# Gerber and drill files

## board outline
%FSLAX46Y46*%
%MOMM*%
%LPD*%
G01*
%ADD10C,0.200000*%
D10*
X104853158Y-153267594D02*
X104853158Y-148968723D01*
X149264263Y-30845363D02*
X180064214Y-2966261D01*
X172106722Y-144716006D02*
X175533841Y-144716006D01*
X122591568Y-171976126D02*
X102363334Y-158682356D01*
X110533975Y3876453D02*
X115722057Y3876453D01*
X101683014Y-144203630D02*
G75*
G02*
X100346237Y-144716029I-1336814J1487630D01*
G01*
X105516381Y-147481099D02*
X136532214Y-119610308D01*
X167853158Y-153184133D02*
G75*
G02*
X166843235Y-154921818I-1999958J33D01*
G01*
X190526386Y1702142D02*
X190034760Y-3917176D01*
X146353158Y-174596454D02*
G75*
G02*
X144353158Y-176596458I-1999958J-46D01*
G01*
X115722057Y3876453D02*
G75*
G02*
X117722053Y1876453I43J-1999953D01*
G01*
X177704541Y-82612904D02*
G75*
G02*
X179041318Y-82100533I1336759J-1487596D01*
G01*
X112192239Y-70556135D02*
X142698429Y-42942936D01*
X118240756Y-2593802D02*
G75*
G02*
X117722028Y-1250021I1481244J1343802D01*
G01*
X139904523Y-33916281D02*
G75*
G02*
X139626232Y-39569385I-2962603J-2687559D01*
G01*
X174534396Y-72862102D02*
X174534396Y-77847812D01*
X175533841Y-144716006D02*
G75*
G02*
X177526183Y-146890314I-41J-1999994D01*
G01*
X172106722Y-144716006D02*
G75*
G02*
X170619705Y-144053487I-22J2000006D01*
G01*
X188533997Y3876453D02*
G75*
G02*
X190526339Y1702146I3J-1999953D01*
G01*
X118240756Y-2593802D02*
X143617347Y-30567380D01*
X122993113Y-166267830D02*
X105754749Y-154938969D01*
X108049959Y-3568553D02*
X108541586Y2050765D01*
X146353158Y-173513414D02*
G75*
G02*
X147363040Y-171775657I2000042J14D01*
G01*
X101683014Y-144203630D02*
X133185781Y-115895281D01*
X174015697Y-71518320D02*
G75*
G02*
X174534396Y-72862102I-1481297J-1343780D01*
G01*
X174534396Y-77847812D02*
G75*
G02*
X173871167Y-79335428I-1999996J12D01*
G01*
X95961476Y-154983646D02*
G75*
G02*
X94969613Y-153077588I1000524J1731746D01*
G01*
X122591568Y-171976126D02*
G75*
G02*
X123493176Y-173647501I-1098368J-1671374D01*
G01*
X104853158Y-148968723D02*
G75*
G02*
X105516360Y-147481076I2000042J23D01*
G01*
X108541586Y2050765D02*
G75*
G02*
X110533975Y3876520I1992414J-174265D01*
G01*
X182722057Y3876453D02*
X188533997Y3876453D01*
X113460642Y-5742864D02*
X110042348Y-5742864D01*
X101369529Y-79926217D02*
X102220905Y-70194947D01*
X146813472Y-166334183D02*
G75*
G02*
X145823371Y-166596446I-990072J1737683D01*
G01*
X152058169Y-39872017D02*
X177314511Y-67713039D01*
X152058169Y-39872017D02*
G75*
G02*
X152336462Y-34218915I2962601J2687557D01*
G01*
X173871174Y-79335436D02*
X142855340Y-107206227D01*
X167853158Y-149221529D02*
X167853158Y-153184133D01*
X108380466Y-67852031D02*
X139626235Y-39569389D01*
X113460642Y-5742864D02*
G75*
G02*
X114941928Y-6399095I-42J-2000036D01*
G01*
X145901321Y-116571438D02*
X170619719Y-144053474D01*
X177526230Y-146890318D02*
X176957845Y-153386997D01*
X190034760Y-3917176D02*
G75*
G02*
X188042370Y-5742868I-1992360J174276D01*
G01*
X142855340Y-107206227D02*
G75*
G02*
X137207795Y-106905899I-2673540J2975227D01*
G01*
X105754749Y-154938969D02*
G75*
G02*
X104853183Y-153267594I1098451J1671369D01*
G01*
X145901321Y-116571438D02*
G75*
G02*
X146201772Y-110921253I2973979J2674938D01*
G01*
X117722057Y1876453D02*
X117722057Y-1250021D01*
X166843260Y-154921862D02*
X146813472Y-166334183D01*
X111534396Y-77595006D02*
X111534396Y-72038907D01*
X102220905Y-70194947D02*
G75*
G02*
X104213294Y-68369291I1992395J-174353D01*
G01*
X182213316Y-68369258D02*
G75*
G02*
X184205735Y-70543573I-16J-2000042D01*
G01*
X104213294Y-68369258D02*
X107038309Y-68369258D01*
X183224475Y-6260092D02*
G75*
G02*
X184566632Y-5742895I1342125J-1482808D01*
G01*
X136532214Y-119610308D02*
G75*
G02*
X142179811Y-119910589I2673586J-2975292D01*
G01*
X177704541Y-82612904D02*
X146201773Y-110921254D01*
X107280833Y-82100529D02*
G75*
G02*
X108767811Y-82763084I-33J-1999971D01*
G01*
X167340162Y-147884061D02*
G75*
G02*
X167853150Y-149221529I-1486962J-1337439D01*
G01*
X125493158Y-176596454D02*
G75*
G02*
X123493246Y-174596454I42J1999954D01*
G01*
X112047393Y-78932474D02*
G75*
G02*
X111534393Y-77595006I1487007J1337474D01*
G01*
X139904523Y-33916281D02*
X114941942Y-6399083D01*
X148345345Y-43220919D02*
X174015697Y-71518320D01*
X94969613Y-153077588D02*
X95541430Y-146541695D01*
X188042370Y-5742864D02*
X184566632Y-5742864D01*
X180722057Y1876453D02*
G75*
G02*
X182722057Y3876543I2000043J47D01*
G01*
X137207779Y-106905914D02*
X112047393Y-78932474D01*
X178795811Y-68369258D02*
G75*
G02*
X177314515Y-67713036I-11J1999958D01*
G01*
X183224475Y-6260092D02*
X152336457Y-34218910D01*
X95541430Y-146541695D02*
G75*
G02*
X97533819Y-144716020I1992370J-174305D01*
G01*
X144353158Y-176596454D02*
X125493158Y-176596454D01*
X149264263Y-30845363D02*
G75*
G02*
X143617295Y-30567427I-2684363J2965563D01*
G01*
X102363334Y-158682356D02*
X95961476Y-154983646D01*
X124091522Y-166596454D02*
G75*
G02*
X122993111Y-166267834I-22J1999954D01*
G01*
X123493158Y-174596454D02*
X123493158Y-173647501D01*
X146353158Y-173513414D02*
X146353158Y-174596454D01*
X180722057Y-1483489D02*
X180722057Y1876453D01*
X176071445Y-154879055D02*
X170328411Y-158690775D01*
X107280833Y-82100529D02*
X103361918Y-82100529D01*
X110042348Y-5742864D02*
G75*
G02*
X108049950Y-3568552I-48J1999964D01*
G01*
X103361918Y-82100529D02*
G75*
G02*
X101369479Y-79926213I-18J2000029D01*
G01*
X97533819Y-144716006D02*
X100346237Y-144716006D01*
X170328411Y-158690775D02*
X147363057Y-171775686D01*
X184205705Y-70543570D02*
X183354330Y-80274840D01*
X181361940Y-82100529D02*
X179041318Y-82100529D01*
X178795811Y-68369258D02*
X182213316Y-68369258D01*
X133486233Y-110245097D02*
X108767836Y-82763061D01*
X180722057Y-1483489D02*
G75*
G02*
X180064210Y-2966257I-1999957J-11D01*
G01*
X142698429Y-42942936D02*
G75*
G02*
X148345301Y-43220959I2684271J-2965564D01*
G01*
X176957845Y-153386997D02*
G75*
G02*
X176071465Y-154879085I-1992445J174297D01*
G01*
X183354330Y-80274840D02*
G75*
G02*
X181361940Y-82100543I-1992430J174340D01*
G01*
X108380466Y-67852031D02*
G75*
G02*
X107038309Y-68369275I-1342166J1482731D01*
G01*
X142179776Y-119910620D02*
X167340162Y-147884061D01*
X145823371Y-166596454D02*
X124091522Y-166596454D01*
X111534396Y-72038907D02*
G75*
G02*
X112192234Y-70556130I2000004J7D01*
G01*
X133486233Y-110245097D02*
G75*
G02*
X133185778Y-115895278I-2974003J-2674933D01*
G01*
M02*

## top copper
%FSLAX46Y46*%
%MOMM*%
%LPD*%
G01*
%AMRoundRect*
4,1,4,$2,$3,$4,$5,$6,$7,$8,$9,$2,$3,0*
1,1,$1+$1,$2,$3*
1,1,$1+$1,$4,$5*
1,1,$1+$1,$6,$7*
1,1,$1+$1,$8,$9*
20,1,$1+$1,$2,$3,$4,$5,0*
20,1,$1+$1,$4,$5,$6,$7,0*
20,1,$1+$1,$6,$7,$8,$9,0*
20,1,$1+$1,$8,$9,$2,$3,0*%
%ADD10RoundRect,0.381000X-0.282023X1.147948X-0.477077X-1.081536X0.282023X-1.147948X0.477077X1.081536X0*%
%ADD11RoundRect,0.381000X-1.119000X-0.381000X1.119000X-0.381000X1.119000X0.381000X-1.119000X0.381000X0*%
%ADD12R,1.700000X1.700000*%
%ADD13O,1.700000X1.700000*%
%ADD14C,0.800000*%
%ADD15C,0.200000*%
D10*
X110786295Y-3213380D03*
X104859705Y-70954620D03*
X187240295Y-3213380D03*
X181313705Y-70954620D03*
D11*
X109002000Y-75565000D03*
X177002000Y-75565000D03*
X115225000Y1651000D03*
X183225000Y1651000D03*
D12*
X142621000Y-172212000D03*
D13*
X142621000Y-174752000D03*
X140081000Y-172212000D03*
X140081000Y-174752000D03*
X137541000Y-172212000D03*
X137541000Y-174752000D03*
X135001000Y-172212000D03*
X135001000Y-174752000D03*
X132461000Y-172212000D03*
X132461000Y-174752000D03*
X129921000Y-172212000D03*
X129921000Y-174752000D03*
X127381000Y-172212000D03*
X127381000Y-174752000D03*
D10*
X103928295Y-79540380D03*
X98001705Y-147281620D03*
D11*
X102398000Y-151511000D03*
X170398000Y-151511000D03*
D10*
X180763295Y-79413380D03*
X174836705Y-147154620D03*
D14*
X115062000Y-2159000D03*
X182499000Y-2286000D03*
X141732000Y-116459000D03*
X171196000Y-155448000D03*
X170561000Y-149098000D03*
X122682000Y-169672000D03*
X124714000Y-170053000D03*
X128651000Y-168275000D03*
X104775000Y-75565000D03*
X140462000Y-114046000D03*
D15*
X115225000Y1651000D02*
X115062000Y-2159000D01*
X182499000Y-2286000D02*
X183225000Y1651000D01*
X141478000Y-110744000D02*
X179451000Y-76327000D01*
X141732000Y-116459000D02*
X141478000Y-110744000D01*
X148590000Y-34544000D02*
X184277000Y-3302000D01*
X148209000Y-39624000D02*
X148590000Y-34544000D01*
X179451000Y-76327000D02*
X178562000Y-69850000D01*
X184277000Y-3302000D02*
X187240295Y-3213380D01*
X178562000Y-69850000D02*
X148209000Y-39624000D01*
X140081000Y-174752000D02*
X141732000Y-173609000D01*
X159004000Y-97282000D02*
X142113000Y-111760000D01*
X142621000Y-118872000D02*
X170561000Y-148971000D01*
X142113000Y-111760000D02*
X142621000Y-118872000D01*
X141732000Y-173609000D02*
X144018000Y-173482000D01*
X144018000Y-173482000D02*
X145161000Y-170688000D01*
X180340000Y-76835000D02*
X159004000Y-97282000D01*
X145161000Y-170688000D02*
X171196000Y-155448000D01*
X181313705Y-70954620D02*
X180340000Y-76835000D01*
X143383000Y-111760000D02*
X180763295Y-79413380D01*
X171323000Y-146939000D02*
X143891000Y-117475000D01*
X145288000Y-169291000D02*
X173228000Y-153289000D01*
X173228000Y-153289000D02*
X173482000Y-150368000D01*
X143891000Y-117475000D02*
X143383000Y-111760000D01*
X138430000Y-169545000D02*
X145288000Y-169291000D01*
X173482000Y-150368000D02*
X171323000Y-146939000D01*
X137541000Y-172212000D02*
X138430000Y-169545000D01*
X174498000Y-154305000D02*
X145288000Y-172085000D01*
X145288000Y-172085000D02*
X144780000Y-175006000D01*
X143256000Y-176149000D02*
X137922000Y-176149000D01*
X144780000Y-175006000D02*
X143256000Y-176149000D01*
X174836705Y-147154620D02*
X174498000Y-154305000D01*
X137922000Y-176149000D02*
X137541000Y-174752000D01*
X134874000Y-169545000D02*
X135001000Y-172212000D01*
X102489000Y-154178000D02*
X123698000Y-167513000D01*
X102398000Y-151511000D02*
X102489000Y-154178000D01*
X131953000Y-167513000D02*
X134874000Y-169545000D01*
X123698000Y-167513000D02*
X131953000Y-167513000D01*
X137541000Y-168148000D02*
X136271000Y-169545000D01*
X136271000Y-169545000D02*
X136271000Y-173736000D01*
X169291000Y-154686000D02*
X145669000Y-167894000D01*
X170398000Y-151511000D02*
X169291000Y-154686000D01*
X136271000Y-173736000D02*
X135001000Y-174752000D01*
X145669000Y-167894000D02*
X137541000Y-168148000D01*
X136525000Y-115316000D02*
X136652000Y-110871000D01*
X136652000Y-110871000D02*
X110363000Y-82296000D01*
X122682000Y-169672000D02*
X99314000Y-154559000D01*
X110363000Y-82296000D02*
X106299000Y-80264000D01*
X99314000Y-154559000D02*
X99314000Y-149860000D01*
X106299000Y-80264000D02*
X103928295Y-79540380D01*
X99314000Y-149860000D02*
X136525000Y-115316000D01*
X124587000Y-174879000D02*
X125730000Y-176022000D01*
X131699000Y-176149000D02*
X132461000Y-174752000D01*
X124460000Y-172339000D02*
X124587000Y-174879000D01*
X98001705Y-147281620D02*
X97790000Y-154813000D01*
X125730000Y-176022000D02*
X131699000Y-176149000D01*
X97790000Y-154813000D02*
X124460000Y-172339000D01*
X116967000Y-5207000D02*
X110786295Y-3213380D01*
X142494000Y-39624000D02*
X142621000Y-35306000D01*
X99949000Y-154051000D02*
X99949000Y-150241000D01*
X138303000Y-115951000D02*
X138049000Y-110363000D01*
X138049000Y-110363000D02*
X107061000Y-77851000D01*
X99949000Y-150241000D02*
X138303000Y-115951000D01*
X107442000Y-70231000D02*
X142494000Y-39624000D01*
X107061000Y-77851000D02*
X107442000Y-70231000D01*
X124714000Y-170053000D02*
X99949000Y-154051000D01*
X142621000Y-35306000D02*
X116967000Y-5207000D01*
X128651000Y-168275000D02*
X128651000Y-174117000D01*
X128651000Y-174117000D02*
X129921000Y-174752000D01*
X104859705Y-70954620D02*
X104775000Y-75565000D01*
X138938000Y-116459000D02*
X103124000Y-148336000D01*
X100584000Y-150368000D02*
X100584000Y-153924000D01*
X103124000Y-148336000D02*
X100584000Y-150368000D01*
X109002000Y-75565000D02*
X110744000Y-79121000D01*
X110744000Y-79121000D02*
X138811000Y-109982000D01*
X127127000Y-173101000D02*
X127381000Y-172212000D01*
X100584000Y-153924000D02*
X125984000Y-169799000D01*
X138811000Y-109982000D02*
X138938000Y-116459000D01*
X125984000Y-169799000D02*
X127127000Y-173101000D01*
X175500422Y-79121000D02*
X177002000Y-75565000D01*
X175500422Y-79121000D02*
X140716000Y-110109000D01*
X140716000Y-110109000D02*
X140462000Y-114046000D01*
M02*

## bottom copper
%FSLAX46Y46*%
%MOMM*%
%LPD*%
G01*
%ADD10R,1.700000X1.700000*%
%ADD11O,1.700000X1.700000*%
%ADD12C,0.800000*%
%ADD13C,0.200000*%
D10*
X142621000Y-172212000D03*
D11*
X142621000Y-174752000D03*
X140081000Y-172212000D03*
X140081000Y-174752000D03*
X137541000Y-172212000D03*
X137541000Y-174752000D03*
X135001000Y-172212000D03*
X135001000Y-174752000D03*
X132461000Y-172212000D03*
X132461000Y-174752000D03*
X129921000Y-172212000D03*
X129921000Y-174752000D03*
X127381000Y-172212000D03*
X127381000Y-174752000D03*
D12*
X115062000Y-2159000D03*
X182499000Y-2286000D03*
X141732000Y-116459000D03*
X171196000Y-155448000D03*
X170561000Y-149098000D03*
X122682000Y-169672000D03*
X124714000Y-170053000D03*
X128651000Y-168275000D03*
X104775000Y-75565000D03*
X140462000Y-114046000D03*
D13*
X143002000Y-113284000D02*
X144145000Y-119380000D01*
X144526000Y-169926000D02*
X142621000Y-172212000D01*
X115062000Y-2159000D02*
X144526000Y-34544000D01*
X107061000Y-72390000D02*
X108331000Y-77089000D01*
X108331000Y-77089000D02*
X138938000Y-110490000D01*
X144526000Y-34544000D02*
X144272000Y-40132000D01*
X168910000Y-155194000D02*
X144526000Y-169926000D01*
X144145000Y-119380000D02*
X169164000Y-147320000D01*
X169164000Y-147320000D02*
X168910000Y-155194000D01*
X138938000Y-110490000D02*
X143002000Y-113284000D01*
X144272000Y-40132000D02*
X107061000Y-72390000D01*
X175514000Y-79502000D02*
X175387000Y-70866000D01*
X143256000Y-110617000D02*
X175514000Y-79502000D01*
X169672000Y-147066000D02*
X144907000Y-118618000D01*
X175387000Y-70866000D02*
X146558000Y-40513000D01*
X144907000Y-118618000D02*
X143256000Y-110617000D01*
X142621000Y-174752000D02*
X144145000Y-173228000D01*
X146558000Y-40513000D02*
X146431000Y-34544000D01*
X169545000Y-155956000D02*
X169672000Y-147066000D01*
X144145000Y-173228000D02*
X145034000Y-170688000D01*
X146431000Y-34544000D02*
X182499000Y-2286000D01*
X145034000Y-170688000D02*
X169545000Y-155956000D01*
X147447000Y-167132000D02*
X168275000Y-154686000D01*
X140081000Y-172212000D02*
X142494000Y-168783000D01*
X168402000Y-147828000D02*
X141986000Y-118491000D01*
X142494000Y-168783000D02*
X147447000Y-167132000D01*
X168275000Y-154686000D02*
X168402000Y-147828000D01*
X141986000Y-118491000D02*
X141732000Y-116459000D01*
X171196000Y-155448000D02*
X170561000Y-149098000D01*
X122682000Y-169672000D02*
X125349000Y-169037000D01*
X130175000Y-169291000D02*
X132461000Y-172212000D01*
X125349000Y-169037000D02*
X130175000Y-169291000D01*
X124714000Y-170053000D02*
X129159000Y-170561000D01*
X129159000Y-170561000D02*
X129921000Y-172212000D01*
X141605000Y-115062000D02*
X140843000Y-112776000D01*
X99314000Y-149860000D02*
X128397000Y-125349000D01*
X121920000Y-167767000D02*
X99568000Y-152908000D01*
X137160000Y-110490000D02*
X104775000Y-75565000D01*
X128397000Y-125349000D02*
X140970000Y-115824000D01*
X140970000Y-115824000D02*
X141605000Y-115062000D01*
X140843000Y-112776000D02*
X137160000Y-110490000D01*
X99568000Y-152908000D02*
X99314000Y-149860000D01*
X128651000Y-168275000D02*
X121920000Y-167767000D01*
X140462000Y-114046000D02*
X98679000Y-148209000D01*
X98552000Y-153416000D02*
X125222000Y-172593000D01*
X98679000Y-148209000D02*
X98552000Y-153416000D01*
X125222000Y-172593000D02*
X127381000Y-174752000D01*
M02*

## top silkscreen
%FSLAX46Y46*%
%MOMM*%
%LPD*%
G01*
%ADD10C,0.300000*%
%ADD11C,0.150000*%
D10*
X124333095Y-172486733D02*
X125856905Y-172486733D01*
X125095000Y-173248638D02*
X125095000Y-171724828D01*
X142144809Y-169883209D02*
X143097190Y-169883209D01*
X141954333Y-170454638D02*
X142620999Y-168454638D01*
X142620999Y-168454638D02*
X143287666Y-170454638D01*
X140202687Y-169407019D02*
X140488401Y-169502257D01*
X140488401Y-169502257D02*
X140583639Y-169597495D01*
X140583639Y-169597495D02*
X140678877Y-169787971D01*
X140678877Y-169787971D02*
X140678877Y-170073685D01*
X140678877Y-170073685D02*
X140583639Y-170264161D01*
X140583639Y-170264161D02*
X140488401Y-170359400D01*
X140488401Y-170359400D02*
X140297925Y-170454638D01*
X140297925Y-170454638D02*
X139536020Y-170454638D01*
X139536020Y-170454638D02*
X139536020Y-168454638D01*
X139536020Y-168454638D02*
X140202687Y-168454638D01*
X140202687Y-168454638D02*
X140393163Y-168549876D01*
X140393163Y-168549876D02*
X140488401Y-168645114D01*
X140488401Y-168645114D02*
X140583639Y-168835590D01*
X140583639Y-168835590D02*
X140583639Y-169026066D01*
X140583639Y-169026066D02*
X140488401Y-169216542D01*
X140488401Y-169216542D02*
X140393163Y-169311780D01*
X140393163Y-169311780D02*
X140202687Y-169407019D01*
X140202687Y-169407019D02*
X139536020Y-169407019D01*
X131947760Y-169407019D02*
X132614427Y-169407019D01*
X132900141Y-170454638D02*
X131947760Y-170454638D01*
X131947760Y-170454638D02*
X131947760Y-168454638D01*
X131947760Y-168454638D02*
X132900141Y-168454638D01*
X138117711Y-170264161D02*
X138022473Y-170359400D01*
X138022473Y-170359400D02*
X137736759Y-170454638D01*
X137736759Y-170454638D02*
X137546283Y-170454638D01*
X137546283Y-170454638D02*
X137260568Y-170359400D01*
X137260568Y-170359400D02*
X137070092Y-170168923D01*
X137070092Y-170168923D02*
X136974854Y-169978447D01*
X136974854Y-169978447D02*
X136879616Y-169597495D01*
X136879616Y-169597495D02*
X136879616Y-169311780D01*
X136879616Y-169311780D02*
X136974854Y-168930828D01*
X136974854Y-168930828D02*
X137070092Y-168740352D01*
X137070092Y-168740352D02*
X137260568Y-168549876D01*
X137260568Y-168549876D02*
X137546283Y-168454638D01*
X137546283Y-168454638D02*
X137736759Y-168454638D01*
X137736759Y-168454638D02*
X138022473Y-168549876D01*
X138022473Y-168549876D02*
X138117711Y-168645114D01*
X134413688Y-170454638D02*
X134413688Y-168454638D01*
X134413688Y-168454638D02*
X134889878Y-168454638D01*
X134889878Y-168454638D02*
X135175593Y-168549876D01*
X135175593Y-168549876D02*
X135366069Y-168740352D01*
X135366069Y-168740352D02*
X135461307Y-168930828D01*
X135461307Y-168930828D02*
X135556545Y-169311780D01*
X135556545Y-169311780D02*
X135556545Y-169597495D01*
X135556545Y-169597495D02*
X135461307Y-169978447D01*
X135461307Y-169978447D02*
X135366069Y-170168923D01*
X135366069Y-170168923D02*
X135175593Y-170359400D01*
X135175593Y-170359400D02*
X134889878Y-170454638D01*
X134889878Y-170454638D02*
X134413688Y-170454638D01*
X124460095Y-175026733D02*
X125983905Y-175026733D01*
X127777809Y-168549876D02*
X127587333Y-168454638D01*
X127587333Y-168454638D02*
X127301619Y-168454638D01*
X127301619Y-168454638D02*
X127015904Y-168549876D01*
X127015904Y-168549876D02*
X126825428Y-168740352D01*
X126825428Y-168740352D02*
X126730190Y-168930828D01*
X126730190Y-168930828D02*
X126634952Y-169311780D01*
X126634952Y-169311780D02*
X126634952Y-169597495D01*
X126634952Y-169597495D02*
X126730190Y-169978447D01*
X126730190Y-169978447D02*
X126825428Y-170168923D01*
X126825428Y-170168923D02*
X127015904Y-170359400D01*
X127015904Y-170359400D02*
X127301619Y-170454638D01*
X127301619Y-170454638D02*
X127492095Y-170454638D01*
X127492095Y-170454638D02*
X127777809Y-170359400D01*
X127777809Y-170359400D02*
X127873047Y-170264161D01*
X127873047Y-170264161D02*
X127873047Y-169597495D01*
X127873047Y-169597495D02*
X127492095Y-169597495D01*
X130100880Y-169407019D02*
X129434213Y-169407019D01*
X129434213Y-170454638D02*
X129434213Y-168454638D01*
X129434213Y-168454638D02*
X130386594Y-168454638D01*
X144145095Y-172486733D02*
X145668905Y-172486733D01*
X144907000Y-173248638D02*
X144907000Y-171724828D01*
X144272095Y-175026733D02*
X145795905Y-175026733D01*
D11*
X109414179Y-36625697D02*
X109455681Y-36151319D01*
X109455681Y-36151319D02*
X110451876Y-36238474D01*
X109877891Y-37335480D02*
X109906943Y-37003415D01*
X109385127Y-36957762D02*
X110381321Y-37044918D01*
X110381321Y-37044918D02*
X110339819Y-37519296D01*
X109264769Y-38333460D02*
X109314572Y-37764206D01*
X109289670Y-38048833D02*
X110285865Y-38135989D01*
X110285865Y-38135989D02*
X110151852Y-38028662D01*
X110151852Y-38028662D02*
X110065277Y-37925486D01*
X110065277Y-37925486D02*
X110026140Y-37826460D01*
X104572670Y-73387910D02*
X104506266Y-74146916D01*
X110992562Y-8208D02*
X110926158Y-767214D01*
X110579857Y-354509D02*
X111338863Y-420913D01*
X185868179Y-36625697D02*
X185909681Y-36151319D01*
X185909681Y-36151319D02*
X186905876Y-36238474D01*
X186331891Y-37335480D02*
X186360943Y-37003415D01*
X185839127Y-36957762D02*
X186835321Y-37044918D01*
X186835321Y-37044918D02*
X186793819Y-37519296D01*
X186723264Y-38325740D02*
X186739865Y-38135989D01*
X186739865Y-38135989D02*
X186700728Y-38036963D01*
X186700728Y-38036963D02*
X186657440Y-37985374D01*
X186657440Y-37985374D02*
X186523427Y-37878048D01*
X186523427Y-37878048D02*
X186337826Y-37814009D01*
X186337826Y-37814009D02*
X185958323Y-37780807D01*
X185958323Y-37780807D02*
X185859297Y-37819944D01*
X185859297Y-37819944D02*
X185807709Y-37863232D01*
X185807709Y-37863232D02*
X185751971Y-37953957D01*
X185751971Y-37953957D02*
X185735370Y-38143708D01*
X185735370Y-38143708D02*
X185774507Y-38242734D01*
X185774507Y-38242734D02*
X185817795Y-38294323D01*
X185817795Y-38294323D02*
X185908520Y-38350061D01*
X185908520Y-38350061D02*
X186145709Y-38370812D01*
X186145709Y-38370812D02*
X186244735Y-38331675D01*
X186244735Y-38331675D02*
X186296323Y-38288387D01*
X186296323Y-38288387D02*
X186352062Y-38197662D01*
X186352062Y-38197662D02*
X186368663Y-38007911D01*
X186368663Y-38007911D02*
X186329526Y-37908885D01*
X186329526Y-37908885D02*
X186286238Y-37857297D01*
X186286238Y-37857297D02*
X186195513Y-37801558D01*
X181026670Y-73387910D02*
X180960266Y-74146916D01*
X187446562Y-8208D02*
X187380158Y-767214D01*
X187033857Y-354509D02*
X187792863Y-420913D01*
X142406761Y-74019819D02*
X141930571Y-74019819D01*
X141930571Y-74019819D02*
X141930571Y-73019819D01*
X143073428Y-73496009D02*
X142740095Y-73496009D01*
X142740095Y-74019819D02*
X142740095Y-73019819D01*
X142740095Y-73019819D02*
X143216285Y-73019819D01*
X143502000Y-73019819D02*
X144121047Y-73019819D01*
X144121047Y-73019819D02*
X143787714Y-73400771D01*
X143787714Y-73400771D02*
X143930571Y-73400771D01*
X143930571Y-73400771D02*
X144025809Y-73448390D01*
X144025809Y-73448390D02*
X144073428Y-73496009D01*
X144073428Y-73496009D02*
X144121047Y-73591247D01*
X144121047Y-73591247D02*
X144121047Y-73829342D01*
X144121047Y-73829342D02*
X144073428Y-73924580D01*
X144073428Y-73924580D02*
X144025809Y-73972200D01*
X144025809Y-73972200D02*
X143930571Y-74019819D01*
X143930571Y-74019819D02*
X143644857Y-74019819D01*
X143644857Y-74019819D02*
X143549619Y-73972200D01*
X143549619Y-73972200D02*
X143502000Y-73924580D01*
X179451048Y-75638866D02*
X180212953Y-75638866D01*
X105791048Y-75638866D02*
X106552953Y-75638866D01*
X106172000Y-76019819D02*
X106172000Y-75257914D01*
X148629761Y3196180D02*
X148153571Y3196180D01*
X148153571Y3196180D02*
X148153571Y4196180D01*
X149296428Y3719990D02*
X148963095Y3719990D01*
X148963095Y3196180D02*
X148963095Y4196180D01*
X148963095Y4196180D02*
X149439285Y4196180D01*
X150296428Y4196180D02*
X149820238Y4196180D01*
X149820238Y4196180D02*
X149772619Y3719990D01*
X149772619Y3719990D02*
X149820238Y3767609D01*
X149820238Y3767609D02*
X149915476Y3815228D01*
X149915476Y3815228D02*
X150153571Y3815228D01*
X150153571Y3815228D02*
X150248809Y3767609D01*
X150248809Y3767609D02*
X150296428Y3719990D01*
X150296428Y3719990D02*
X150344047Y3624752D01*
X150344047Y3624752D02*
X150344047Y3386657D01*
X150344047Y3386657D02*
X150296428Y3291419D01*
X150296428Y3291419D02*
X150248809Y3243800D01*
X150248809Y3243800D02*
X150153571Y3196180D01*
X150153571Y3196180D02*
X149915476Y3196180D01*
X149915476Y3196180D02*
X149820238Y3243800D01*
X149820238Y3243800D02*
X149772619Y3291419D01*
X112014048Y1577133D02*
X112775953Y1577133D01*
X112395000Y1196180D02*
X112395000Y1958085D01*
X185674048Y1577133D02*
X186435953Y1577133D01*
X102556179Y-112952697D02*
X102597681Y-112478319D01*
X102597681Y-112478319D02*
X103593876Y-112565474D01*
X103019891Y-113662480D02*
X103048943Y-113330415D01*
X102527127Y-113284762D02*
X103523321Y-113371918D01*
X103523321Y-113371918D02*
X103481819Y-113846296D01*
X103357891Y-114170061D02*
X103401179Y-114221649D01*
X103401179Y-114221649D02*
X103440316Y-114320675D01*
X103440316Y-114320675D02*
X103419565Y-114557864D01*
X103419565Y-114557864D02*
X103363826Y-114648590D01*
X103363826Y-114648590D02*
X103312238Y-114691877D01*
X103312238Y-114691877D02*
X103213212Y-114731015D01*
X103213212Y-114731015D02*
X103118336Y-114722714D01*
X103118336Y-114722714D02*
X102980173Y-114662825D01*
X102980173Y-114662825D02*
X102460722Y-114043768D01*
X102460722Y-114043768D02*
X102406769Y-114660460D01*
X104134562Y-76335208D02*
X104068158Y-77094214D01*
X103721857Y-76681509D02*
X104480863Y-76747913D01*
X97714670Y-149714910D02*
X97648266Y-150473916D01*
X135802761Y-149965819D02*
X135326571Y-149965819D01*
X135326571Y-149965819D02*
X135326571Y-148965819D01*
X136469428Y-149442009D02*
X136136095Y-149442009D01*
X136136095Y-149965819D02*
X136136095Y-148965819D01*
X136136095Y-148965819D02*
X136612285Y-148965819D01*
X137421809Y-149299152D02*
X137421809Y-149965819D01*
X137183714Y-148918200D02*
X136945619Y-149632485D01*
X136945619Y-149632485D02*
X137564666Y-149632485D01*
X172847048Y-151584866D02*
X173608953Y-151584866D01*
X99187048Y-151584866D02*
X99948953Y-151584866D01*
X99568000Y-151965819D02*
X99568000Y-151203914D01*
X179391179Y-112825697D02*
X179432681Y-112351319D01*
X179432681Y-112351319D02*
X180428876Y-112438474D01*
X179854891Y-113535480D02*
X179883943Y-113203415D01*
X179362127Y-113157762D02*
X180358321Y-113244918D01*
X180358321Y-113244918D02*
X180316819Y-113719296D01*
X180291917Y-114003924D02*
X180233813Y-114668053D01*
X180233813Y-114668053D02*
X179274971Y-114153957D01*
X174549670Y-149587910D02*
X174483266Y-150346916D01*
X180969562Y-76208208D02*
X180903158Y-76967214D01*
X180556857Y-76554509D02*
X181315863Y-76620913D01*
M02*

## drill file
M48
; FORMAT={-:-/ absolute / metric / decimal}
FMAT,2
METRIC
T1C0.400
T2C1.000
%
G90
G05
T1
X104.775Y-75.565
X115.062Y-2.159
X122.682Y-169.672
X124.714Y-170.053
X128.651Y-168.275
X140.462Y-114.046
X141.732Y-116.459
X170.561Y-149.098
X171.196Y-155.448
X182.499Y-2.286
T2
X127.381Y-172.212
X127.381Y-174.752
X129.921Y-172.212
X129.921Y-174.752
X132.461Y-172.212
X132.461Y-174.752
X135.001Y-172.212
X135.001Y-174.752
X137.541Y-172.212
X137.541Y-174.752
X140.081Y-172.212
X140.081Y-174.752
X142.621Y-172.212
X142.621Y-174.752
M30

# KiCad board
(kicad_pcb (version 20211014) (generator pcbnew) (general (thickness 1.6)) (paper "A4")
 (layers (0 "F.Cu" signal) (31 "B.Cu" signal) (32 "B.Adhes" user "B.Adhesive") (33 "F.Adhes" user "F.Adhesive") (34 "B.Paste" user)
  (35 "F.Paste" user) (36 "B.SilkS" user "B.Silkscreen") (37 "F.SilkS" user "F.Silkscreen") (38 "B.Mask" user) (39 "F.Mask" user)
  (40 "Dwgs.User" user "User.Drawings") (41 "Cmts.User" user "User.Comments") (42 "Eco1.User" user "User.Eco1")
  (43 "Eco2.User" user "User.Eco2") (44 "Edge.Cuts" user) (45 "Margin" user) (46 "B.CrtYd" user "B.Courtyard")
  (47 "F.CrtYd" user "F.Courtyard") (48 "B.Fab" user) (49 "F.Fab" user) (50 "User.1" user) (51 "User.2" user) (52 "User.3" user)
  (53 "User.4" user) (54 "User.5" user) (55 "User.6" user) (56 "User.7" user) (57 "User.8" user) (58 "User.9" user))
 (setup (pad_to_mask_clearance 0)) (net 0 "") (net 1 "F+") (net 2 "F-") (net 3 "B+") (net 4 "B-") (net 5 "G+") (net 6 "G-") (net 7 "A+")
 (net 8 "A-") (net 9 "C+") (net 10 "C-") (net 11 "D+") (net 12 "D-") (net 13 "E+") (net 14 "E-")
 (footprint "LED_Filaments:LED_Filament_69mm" (layer "F.Cu") (at 107.823 37.084 -95)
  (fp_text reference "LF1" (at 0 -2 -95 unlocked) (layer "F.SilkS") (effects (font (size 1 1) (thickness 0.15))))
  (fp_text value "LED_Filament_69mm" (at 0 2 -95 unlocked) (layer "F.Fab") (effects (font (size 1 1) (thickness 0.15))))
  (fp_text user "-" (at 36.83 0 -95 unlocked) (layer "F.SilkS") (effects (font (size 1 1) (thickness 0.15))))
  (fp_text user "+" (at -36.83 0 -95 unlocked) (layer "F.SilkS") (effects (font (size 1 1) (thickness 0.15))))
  (pad "1" smd roundrect (at -34 0 265) (size 3 1.524) (layers "F.Cu" "F.Paste" "F.Mask") (roundrect_rratio 0.25) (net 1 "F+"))
  (pad "2" smd roundrect (at 34 0 265) (size 3 1.524) (layers "F.Cu" "F.Paste" "F.Mask") (roundrect_rratio 0.25) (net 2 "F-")))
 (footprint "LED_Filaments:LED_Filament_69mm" (layer "F.Cu") (at 184.277 37.084 -95)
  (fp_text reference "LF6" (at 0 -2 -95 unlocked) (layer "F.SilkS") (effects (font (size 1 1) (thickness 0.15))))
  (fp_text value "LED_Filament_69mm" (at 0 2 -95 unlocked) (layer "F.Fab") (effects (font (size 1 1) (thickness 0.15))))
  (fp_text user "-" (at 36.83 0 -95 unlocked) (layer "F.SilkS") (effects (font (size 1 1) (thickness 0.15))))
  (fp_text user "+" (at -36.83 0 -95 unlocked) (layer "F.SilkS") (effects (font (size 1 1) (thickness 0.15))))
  (pad "1" smd roundrect (at -34 0 265) (size 3 1.524) (layers "F.Cu" "F.Paste" "F.Mask") (roundrect_rratio 0.25) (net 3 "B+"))
  (pad "2" smd roundrect (at 34 0 265) (size 3 1.524) (layers "F.Cu" "F.Paste" "F.Mask") (roundrect_rratio 0.25) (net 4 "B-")))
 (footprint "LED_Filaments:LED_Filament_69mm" (layer "F.Cu") (at 143.002 75.565)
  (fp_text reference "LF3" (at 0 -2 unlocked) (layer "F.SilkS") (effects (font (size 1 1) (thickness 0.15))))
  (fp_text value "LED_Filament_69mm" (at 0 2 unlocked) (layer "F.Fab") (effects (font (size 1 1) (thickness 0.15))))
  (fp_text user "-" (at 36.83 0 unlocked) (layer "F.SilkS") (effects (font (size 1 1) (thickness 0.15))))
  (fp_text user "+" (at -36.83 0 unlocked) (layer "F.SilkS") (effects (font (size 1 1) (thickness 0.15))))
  (pad "1" smd roundrect (at -34 0) (size 3 1.524) (layers "F.Cu" "F.Paste" "F.Mask") (roundrect_rratio 0.25) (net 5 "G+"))
  (pad "2" smd roundrect (at 34 0) (size 3 1.524) (layers "F.Cu" "F.Paste" "F.Mask") (roundrect_rratio 0.25) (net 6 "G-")))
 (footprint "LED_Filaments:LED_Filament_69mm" (layer "F.Cu") (at 149.225 -1.651)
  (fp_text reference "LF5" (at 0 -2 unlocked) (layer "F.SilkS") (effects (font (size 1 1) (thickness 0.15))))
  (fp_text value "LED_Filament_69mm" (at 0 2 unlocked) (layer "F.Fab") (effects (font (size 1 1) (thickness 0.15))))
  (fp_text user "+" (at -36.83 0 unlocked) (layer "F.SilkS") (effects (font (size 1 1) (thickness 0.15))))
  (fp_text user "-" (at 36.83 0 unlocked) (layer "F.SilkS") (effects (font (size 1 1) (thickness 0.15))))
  (pad "1" smd roundrect (at -34 0) (size 3 1.524) (layers "F.Cu" "F.Paste" "F.Mask") (roundrect_rratio 0.25) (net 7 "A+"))
  (pad "2" smd roundrect (at 34 0) (size 3 1.524) (layers "F.Cu" "F.Paste" "F.Mask") (roundrect_rratio 0.25) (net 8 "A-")))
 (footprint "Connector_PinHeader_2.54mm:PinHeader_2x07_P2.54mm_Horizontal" (layer "F.Cu") (at 142.621 172.212 -90)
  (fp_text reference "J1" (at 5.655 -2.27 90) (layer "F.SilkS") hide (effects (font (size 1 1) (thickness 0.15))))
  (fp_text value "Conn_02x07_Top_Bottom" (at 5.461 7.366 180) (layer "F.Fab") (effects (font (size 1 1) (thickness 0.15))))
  (pad "1" thru_hole rect (at 0 0 270) (size 1.7 1.7) (drill 1) (layers *.Cu *.Mask) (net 7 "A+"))
  (pad "2" thru_hole oval (at 2.54 0 270) (size 1.7 1.7) (drill 1) (layers *.Cu *.Mask) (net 8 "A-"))
  (pad "3" thru_hole oval (at 0 2.54 270) (size 1.7 1.7) (drill 1) (layers *.Cu *.Mask) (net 3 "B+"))
  (pad "4" thru_hole oval (at 2.54 2.54 270) (size 1.7 1.7) (drill 1) (layers *.Cu *.Mask) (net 4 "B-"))
  (pad "5" thru_hole oval (at 0 5.08 270) (size 1.7 1.7) (drill 1) (layers *.Cu *.Mask) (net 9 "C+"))
  (pad "6" thru_hole oval (at 2.54 5.08 270) (size 1.7 1.7) (drill 1) (layers *.Cu *.Mask) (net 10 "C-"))
  (pad "7" thru_hole oval (at 0 7.62 270) (size 1.7 1.7) (drill 1) (layers *.Cu *.Mask) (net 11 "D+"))
  (pad "8" thru_hole oval (at 2.54 7.62 270) (size 1.7 1.7) (drill 1) (layers *.Cu *.Mask) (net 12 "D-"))
  (pad "9" thru_hole oval (at 0 10.16 270) (size 1.7 1.7) (drill 1) (layers *.Cu *.Mask) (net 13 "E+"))
  (pad "10" thru_hole oval (at 2.54 10.16 270) (size 1.7 1.7) (drill 1) (layers *.Cu *.Mask) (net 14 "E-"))
  (pad "11" thru_hole oval (at 0 12.7 270) (size 1.7 1.7) (drill 1) (layers *.Cu *.Mask) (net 1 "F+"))
  (pad "12" thru_hole oval (at 2.54 12.7 270) (size 1.7 1.7) (drill 1) (layers *.Cu *.Mask) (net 2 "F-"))
  (pad "13" thru_hole oval (at 0 15.24 270) (size 1.7 1.7) (drill 1) (layers *.Cu *.Mask) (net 5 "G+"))
  (pad "14" thru_hole oval (at 2.54 15.24 270) (size 1.7 1.7) (drill 1) (layers *.Cu *.Mask) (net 6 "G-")))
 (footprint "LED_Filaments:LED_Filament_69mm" (layer "F.Cu") (at 100.965 113.411 -95)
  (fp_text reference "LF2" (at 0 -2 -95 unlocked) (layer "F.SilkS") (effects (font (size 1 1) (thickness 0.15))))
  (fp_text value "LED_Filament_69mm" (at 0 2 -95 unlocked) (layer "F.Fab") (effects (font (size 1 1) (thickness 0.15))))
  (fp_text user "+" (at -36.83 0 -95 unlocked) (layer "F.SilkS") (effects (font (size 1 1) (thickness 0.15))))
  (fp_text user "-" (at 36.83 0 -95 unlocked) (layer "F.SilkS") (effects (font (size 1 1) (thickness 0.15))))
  (pad "1" smd roundrect (at -34 0 265) (size 3 1.524) (layers "F.Cu" "F.Paste" "F.Mask") (roundrect_rratio 0.25) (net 13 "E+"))
  (pad "2" smd roundrect (at 34 0 265) (size 3 1.524) (layers "F.Cu" "F.Paste" "F.Mask") (roundrect_rratio 0.25) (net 14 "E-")))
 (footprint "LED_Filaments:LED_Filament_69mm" (layer "F.Cu") (at 136.398 151.511)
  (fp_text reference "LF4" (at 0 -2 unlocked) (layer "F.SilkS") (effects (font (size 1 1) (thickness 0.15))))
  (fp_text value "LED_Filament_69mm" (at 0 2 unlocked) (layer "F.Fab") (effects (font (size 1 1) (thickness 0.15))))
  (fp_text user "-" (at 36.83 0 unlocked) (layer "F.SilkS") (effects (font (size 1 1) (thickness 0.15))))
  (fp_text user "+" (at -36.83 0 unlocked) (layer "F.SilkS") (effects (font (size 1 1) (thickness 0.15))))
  (pad "1" smd roundrect (at -34 0) (size 3 1.524) (layers "F.Cu" "F.Paste" "F.Mask") (roundrect_rratio 0.25) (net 11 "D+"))
  (pad "2" smd roundrect (at 34 0) (size 3 1.524) (layers "F.Cu" "F.Paste" "F.Mask") (roundrect_rratio 0.25) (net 12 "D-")))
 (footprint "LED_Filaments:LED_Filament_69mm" (layer "F.Cu") (at 177.8 113.284 -95)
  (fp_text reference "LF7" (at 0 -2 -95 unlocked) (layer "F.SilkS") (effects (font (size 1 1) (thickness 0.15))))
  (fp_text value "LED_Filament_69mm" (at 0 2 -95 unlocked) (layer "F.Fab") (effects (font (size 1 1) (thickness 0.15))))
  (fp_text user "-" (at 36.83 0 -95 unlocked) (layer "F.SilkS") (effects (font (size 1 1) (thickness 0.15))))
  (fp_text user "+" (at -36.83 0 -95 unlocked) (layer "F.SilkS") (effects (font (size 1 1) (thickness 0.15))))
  (pad "1" smd roundrect (at -34 0 265) (size 3 1.524) (layers "F.Cu" "F.Paste" "F.Mask") (roundrect_rratio 0.25) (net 9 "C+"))
  (pad "2" smd roundrect (at 34 0 265) (size 3 1.524) (layers "F.Cu" "F.Paste" "F.Mask") (roundrect_rratio 0.25) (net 10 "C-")))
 (gr_line (start 104.853158 153.267594) (end 104.853158 148.968723) (layer "Edge.Cuts") (width 0.2))
 (gr_line (start 149.264263 30.845363) (end 180.064214 2.966261) (layer "Edge.Cuts") (width 0.2))
 (gr_line (start 172.106722 144.716006) (end 175.533841 144.716006) (layer "Edge.Cuts") (width 0.2))
 (gr_line (start 122.591568 171.976126) (end 102.363334 158.682356) (layer "Edge.Cuts") (width 0.2))
 (gr_line (start 110.533975 -3.876453) (end 115.722057 -3.876453) (layer "Edge.Cuts") (width 0.2))
 (gr_arc (start 101.683014 144.20363) (mid 101.062041 144.583524) (end 100.346237 144.716006) (layer "Edge.Cuts") (width 0.2))
 (gr_line (start 105.516381 147.481099) (end 136.532214 119.610308) (layer "Edge.Cuts") (width 0.2))
 (gr_arc (start 167.853158 153.184133) (mid 167.582349 154.189071) (end 166.84326 154.921862) (layer "Edge.Cuts") (width 0.2))
 (gr_line (start 190.526386 -1.702142) (end 190.03476 3.917176) (layer "Edge.Cuts") (width 0.2))
 (gr_arc (start 146.353158 174.596454) (mid 145.767372 176.010668) (end 144.353158 176.596454) (layer "Edge.Cuts") (width 0.2))
 (gr_arc (start 115.722057 -3.876453) (mid 117.136271 -3.290667) (end 117.722057 -1.876453) (layer "Edge.Cuts") (width 0.2))
 (gr_arc (start 177.704541 82.612904) (mid 178.325514 82.233011) (end 179.041318 82.100529) (layer "Edge.Cuts") (width 0.2))
 (gr_line (start 112.192239 70.556135) (end 142.698429 42.942936) (layer "Edge.Cuts") (width 0.2))
 (gr_arc (start 118.240756 2.593802) (mid 117.856232 1.970229) (end 117.722057 1.250021) (layer "Edge.Cuts") (width 0.2))
 (gr_arc (start 139.904523 33.916281) (mid 140.937083 36.800515) (end 139.626235 39.569389) (layer "Edge.Cuts") (width 0.2))
 (gr_line (start 174.534396 72.862102) (end 174.534396 77.847812) (layer "Edge.Cuts") (width 0.2))
 (gr_arc (start 175.533841 144.716006) (mid 177.008396 145.364826) (end 177.52623 146.890318) (layer "Edge.Cuts") (width 0.2))
 (gr_arc (start 172.106722 144.716006) (mid 171.292761 144.54288) (end 170.619719 144.053474) (layer "Edge.Cuts") (width 0.2))
 (gr_arc (start 188.533997 -3.876453) (mid 190.008552 -3.227634) (end 190.526386 -1.702142) (layer "Edge.Cuts") (width 0.2))
 (gr_line (start 118.240756 2.593802) (end 143.617347 30.56738) (layer "Edge.Cuts") (width 0.2))
 (gr_line (start 122.993113 166.26783) (end 105.754749 154.938969) (layer "Edge.Cuts") (width 0.2))
 (gr_line (start 108.049959 3.568553) (end 108.541586 -2.050765) (layer "Edge.Cuts") (width 0.2))
 (gr_arc (start 146.353158 173.513414) (mid 146.623968 172.508477) (end 147.363057 171.775686) (layer "Edge.Cuts") (width 0.2))
 (gr_line (start 101.683014 144.20363) (end 133.185781 115.895281) (layer "Edge.Cuts") (width 0.2))
 (gr_arc (start 174.015697 71.51832) (mid 174.400221 72.141894) (end 174.534396 72.862102) (layer "Edge.Cuts") (width 0.2))
 (gr_arc (start 174.534396 77.847812) (mid 174.361081 78.662197) (end 173.871174 79.335436) (layer "Edge.Cuts") (width 0.2))
 (gr_arc (start 95.961476 154.983646) (mid 95.187841 154.175127) (end 94.969613 153.077588) (layer "Edge.Cuts") (width 0.2))
 (gr_arc (start 122.591568 171.976126) (mid 123.253388 172.69798) (end 123.493158 173.647501) (layer "Edge.Cuts") (width 0.2))
 (gr_arc (start 104.853158 148.968723) (mid 105.026474 148.154338) (end 105.516381 147.481099) (layer "Edge.Cuts") (width 0.2))
 (gr_arc (start 108.541586 -2.050765) (mid 109.182795 -3.351008) (end 110.533975 -3.876453) (layer "Edge.Cuts") (width 0.2))
 (gr_line (start 182.722057 -3.876453) (end 188.533997 -3.876453) (layer "Edge.Cuts") (width 0.2))
 (gr_line (start 113.460642 5.742864) (end 110.042348 5.742864) (layer "Edge.Cuts") (width 0.2))
 (gr_line (start 101.369529 79.926217) (end 102.220905 70.194947) (layer "Edge.Cuts") (width 0.2))
 (gr_arc (start 146.813472 166.334183) (mid 146.335496 166.529775) (end 145.823371 166.596454) (layer "Edge.Cuts") (width 0.2))
 (gr_line (start 152.058169 39.872017) (end 177.314511 67.713039) (layer "Edge.Cuts") (width 0.2))
 (gr_arc (start 152.058169 39.872017) (mid 151.025609 36.987783) (end 152.336457 34.21891) (layer "Edge.Cuts") (width 0.2))
 (gr_line (start 173.871174 79.335436) (end 142.85534 107.206227) (layer "Edge.Cuts") (width 0.2))
 (gr_line (start 167.853158 149.221529) (end 167.853158 153.184133) (layer "Edge.Cuts") (width 0.2))
 (gr_line (start 108.380466 67.852031) (end 139.626235 39.569389) (layer "Edge.Cuts") (width 0.2))
 (gr_arc (start 113.460642 5.742864) (mid 114.270715 5.914264) (end 114.941942 6.399083) (layer "Edge.Cuts") (width 0.2))
 (gr_line (start 145.901321 116.571438) (end 170.619719 144.053474) (layer "Edge.Cuts") (width 0.2))
 (gr_line (start 177.52623 146.890318) (end 176.957845 153.386997) (layer "Edge.Cuts") (width 0.2))
 (gr_arc (start 190.03476 3.917176) (mid 189.393551 5.21742) (end 188.04237 5.742864) (layer "Edge.Cuts") (width 0.2))
 (gr_arc (start 142.85534 107.206227) (mid 139.969383 108.225335) (end 137.207779 106.905914) (layer "Edge.Cuts") (width 0.2))
 (gr_arc (start 105.754749 154.938969) (mid 105.092929 154.217115) (end 104.853158 153.267594) (layer "Edge.Cuts") (width 0.2))
 (gr_arc (start 145.901321 116.571438) (mid 144.880972 113.6841) (end 146.201773 110.921254) (layer "Edge.Cuts") (width 0.2))
 (gr_line (start 117.722057 -1.876453) (end 117.722057 1.250021) (layer "Edge.Cuts") (width 0.2))
 (gr_line (start 166.84326 154.921862) (end 146.813472 166.334183) (layer "Edge.Cuts") (width 0.2))
 (gr_line (start 111.534396 77.595006) (end 111.534396 72.038907) (layer "Edge.Cuts") (width 0.2))
 (gr_arc (start 102.220905 70.194947) (mid 102.862113 68.894703) (end 104.213294 68.369258) (layer "Edge.Cuts") (width 0.2))
 (gr_arc (start 182.213316 68.369258) (mid 183.687871 69.018078) (end 184.205705 70.54357) (layer "Edge.Cuts") (width 0.2))
 (gr_line (start 104.213294 68.369258) (end 107.038309 68.369258) (layer "Edge.Cuts") (width 0.2))
 (gr_arc (start 183.224475 6.260092) (mid 183.847447 5.876646) (end 184.566632 5.742864) (layer "Edge.Cuts") (width 0.2))
 (gr_arc (start 136.532214 119.610308) (mid 139.418171 118.5912) (end 142.179776 119.91062) (layer "Edge.Cuts") (width 0.2))
 (gr_line (start 177.704541 82.612904) (end 146.201773 110.921254) (layer "Edge.Cuts") (width 0.2))
 (gr_arc (start 107.280833 82.100529) (mid 108.094793 82.273655) (end 108.767836 82.763061) (layer "Edge.Cuts") (width 0.2))
 (gr_arc (start 167.340162 147.884061) (mid 167.72051 148.505291) (end 167.853158 149.221529) (layer "Edge.Cuts") (width 0.2))
 (gr_arc (start 125.493158 176.596454) (mid 124.078944 176.010668) (end 123.493158 174.596454) (layer "Edge.Cuts") (width 0.2))
 (gr_arc (start 112.047393 78.932474) (mid 111.667044 78.311244) (end 111.534396 77.595006) (layer "Edge.Cuts") (width 0.2))
 (gr_line (start 139.904523 33.916281) (end 114.941942 6.399083) (layer "Edge.Cuts") (width 0.2))
 (gr_line (start 148.345345 43.220919) (end 174.015697 71.51832) (layer "Edge.Cuts") (width 0.2))
 (gr_line (start 94.969613 153.077588) (end 95.54143 146.541695) (layer "Edge.Cuts") (width 0.2))
 (gr_line (start 188.04237 5.742864) (end 184.566632 5.742864) (layer "Edge.Cuts") (width 0.2))
 (gr_arc (start 180.722057 -1.876453) (mid 181.307843 -3.290667) (end 182.722057 -3.876453) (layer "Edge.Cuts") (width 0.2))
 (gr_line (start 137.207779 106.905914) (end 112.047393 78.932474) (layer "Edge.Cuts") (width 0.2))
 (gr_arc (start 178.795811 68.369258) (mid 177.985738 68.197859) (end 177.314511 67.713039) (layer "Edge.Cuts") (width 0.2))
 (gr_line (start 183.224475 6.260092) (end 152.336457 34.21891) (layer "Edge.Cuts") (width 0.2))
 (gr_arc (start 95.54143 146.541695) (mid 96.182638 145.241451) (end 97.533819 144.716006) (layer "Edge.Cuts") (width 0.2))
 (gr_line (start 144.353158 176.596454) (end 125.493158 176.596454) (layer "Edge.Cuts") (width 0.2))
 (gr_arc (start 149.264263 30.845363) (mid 146.383277 31.87498) (end 143.617347 30.56738) (layer "Edge.Cuts") (width 0.2))
 (gr_line (start 102.363334 158.682356) (end 95.961476 154.983646) (layer "Edge.Cuts") (width 0.2))
 (gr_arc (start 124.091522 166.596454) (mid 123.518264 166.512538) (end 122.993113 166.26783) (layer "Edge.Cuts") (width 0.2))
 (gr_line (start 123.493158 174.596454) (end 123.493158 173.647501) (layer "Edge.Cuts") (width 0.2))
 (gr_line (start 146.353158 173.513414) (end 146.353158 174.596454) (layer "Edge.Cuts") (width 0.2))
 (gr_line (start 180.722057 1.483489) (end 180.722057 -1.876453) (layer "Edge.Cuts") (width 0.2))
 (gr_line (start 176.071445 154.879055) (end 170.328411 158.690775) (layer "Edge.Cuts") (width 0.2))
 (gr_line (start 107.280833 82.100529) (end 103.361918 82.100529) (layer "Edge.Cuts") (width 0.2))
 (gr_arc (start 110.042348 5.742864) (mid 108.567793 5.094045) (end 108.049959 3.568553) (layer "Edge.Cuts") (width 0.2))
 (gr_arc (start 103.361918 82.100529) (mid 101.887364 81.451709) (end 101.369529 79.926217) (layer "Edge.Cuts") (width 0.2))
 (gr_line (start 97.533819 144.716006) (end 100.346237 144.716006) (layer "Edge.Cuts") (width 0.2))
 (gr_line (start 170.328411 158.690775) (end 147.363057 171.775686) (layer "Edge.Cuts") (width 0.2))
 (gr_line (start 184.205705 70.54357) (end 183.35433 80.27484) (layer "Edge.Cuts") (width 0.2))
 (gr_line (start 181.36194 82.100529) (end 179.041318 82.100529) (layer "Edge.Cuts") (width 0.2))
 (gr_line (start 178.795811 68.369258) (end 182.213316 68.369258) (layer "Edge.Cuts") (width 0.2))
 (gr_line (start 133.486233 110.245097) (end 108.767836 82.763061) (layer "Edge.Cuts") (width 0.2))
 (gr_arc (start 180.722057 1.483489) (mid 180.550213 2.294564) (end 180.064214 2.966261) (layer "Edge.Cuts") (width 0.2))
 (gr_arc (start 142.698429 42.942936) (mid 145.579415 41.913319) (end 148.345345 43.220919) (layer "Edge.Cuts") (width 0.2))
 (gr_arc (start 176.957845 153.386997) (mid 176.684916 154.234181) (end 176.071445 154.879055) (layer "Edge.Cuts") (width 0.2))
 (gr_arc (start 183.35433 80.27484) (mid 182.713121 81.575084) (end 181.36194 82.100529) (layer "Edge.Cuts") (width 0.2))
 (gr_arc (start 108.380466 67.852031) (mid 107.757494 68.235477) (end 107.038309 68.369258) (layer "Edge.Cuts") (width 0.2))
 (gr_line (start 142.179776 119.91062) (end 167.340162 147.884061) (layer "Edge.Cuts") (width 0.2))
 (gr_line (start 145.823371 166.596454) (end 124.091522 166.596454) (layer "Edge.Cuts") (width 0.2))
 (gr_arc (start 111.534396 72.038907) (mid 111.70624 71.227832) (end 112.192239 70.556135) (layer "Edge.Cuts") (width 0.2))
 (gr_arc (start 133.486233 110.245097) (mid 134.506583 113.132435) (end 133.185781 115.895281) (layer "Edge.Cuts") (width 0.2))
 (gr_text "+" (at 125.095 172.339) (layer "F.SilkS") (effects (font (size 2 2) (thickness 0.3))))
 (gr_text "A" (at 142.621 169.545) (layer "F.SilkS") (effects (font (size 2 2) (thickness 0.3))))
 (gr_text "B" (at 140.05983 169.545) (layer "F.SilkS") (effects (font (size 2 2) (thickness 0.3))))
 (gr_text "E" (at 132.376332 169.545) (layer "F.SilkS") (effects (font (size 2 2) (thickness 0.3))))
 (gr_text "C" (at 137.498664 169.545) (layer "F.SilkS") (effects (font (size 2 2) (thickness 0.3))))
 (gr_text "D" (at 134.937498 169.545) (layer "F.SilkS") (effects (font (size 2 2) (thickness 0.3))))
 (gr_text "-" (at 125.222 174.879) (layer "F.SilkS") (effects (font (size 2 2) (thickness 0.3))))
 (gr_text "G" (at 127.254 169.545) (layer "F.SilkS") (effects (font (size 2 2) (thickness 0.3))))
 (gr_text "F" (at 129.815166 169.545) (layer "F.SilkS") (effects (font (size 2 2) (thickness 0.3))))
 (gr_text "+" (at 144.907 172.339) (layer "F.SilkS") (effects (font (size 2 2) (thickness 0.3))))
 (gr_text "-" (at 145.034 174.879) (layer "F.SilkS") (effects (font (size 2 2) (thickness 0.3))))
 (segment (start 115.225 -1.651) (end 115.062 2.159) (width 0.2) (layer "F.Cu") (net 7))
 (via (at 115.062 2.159) (size 0.8) (drill 0.4) (layers "F.Cu" "B.Cu") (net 7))
 (segment (start 143.002 113.284) (end 144.145 119.38) (width 0.2) (layer "B.Cu") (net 7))
 (segment (start 144.526 169.926) (end 142.621 172.212) (width 0.2) (layer "B.Cu") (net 7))
 (segment (start 115.062 2.159) (end 144.526 34.544) (width 0.2) (layer "B.Cu") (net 7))
 (segment (start 107.061 72.39) (end 108.331 77.089) (width 0.2) (layer "B.Cu") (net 7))
 (segment (start 108.331 77.089) (end 138.938 110.49) (width 0.2) (layer "B.Cu") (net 7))
 (segment (start 144.526 34.544) (end 144.272 40.132) (width 0.2) (layer "B.Cu") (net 7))
 (segment (start 168.91 155.194) (end 144.526 169.926) (width 0.2) (layer "B.Cu") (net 7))
 (segment (start 144.145 119.38) (end 169.164 147.32) (width 0.2) (layer "B.Cu") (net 7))
 (segment (start 169.164 147.32) (end 168.91 155.194) (width 0.2) (layer "B.Cu") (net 7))
 (segment (start 138.938 110.49) (end 143.002 113.284) (width 0.2) (layer "B.Cu") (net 7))
 (segment (start 144.272 40.132) (end 107.061 72.39) (width 0.2) (layer "B.Cu") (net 7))
 (segment (start 182.499 2.286) (end 183.225 -1.651) (width 0.2) (layer "F.Cu") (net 8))
 (via (at 182.499 2.286) (size 0.8) (drill 0.4) (layers "F.Cu" "B.Cu") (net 8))
 (segment (start 175.514 79.502) (end 175.387 70.866) (width 0.2) (layer "B.Cu") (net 8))
 (segment (start 143.256 110.617) (end 175.514 79.502) (width 0.2) (layer "B.Cu") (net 8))
 (segment (start 169.672 147.066) (end 144.907 118.618) (width 0.2) (layer "B.Cu") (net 8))
 (segment (start 175.387 70.866) (end 146.558 40.513) (width 0.2) (layer "B.Cu") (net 8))
 (segment (start 144.907 118.618) (end 143.256 110.617) (width 0.2) (layer "B.Cu") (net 8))
 (segment (start 142.621 174.752) (end 144.145 173.228) (width 0.2) (layer "B.Cu") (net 8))
 (segment (start 146.558 40.513) (end 146.431 34.544) (width 0.2) (layer "B.Cu") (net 8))
 (segment (start 169.545 155.956) (end 169.672 147.066) (width 0.2) (layer "B.Cu") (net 8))
 (segment (start 144.145 173.228) (end 145.034 170.688) (width 0.2) (layer "B.Cu") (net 8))
 (segment (start 146.431 34.544) (end 182.499 2.286) (width 0.2) (layer "B.Cu") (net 8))
 (segment (start 145.034 170.688) (end 169.545 155.956) (width 0.2) (layer "B.Cu") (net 8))
 (segment (start 141.478 110.744) (end 179.451 76.327) (width 0.2) (layer "F.Cu") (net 3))
 (segment (start 141.732 116.459) (end 141.478 110.744) (width 0.2) (layer "F.Cu") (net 3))
 (segment (start 148.59 34.544) (end 184.277 3.302) (width 0.2) (layer "F.Cu") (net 3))
 (segment (start 148.209 39.624) (end 148.59 34.544) (width 0.2) (layer "F.Cu") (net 3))
 (segment (start 179.451 76.327) (end 178.562 69.85) (width 0.2) (layer "F.Cu") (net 3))
 (segment (start 184.277 3.302) (end 187.240295 3.21338) (width 0.2) (layer "F.Cu") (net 3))
 (segment (start 178.562 69.85) (end 148.209 39.624) (width 0.2) (layer "F.Cu") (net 3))
 (via (at 141.732 116.459) (size 0.8) (drill 0.4) (layers "F.Cu" "B.Cu") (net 3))
 (segment (start 147.447 167.132) (end 168.275 154.686) (width 0.2) (layer "B.Cu") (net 3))
 (segment (start 140.081 172.212) (end 142.494 168.783) (width 0.2) (layer "B.Cu") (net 3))
 (segment (start 168.402 147.828) (end 141.986 118.491) (width 0.2) (layer "B.Cu") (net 3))
 (segment (start 142.494 168.783) (end 147.447 167.132) (width 0.2) (layer "B.Cu") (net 3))
 (segment (start 168.275 154.686) (end 168.402 147.828) (width 0.2) (layer "B.Cu") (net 3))
 (segment (start 141.986 118.491) (end 141.732 116.459) (width 0.2) (layer "B.Cu") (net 3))
 (segment (start 140.081 174.752) (end 141.732 173.609) (width 0.2) (layer "F.Cu") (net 4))
 (segment (start 159.004 97.282) (end 142.113 111.76) (width 0.2) (layer "F.Cu") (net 4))
 (segment (start 142.621 118.872) (end 170.561 148.971) (width 0.2) (layer "F.Cu") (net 4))
 (segment (start 142.113 111.76) (end 142.621 118.872) (width 0.2) (layer "F.Cu") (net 4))
 (segment (start 141.732 173.609) (end 144.018 173.482) (width 0.2) (layer "F.Cu") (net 4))
 (segment (start 144.018 173.482) (end 145.161 170.688) (width 0.2) (layer "F.Cu") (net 4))
 (segment (start 180.34 76.835) (end 159.004 97.282) (width 0.2) (layer "F.Cu") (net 4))
 (segment (start 145.161 170.688) (end 171.196 155.448) (width 0.2) (layer "F.Cu") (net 4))
 (segment (start 181.313705 70.95462) (end 180.34 76.835) (width 0.2) (layer "F.Cu") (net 4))
 (via (at 171.196 155.448) (size 0.8) (drill 0.4) (layers "F.Cu" "B.Cu") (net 4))
 (via (at 170.561 149.098) (size 0.8) (drill 0.4) (layers "F.Cu" "B.Cu") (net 4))
 (segment (start 171.196 155.448) (end 170.561 149.098) (width 0.2) (layer "B.Cu") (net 4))
 (segment (start 143.383 111.76) (end 180.763295 79.41338) (width 0.2) (layer "F.Cu") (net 9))
 (segment (start 171.323 146.939) (end 143.891 117.475) (width 0.2) (layer "F.Cu") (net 9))
 (segment (start 145.288 169.291) (end 173.228 153.289) (width 0.2) (layer "F.Cu") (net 9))
 (segment (start 173.228 153.289) (end 173.482 150.368) (width 0.2) (layer "F.Cu") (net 9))
 (segment (start 143.891 117.475) (end 143.383 111.76) (width 0.2) (layer "F.Cu") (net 9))
 (segment (start 138.43 169.545) (end 145.288 169.291) (width 0.2) (layer "F.Cu") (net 9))
 (segment (start 173.482 150.368) (end 171.323 146.939) (width 0.2) (layer "F.Cu") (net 9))
 (segment (start 137.541 172.212) (end 138.43 169.545) (width 0.2) (layer "F.Cu") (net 9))
 (segment (start 174.498 154.305) (end 145.288 172.085) (width 0.2) (layer "F.Cu") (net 10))
 (segment (start 145.288 172.085) (end 144.78 175.006) (width 0.2) (layer "F.Cu") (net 10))
 (segment (start 143.256 176.149) (end 137.922 176.149) (width 0.2) (layer "F.Cu") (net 10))
 (segment (start 144.78 175.006) (end 143.256 176.149) (width 0.2) (layer "F.Cu") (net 10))
 (segment (start 174.836705 147.15462) (end 174.498 154.305) (width 0.2) (layer "F.Cu") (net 10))
 (segment (start 137.922 176.149) (end 137.541 174.752) (width 0.2) (layer "F.Cu") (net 10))
 (segment (start 134.874 169.545) (end 135.001 172.212) (width 0.2) (layer "F.Cu") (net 11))
 (segment (start 102.489 154.178) (end 123.698 167.513) (width 0.2) (layer "F.Cu") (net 11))
 (segment (start 102.398 151.511) (end 102.489 154.178) (width 0.2) (layer "F.Cu") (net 11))
 (segment (start 131.953 167.513) (end 134.874 169.545) (width 0.2) (layer "F.Cu") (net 11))
 (segment (start 123.698 167.513) (end 131.953 167.513) (width 0.2) (layer "F.Cu") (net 11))
 (segment (start 137.541 168.148) (end 136.271 169.545) (width 0.2) (layer "F.Cu") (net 12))
 (segment (start 136.271 169.545) (end 136.271 173.736) (width 0.2) (layer "F.Cu") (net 12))
 (segment (start 169.291 154.686) (end 145.669 167.894) (width 0.2) (layer "F.Cu") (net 12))
 (segment (start 170.398 151.511) (end 169.291 154.686) (width 0.2) (layer "F.Cu") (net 12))
 (segment (start 136.271 173.736) (end 135.001 174.752) (width 0.2) (layer "F.Cu") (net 12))
 (segment (start 145.669 167.894) (end 137.541 168.148) (width 0.2) (layer "F.Cu") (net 12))
 (segment (start 136.525 115.316) (end 136.652 110.871) (width 0.2) (layer "F.Cu") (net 13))
 (segment (start 136.652 110.871) (end 110.363 82.296) (width 0.2) (layer "F.Cu") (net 13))
 (segment (start 122.682 169.672) (end 99.314 154.559) (width 0.2) (layer "F.Cu") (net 13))
 (segment (start 110.363 82.296) (end 106.299 80.264) (width 0.2) (layer "F.Cu") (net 13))
 (segment (start 99.314 154.559) (end 99.314 149.86) (width 0.2) (layer "F.Cu") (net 13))
 (segment (start 106.299 80.264) (end 103.928295 79.54038) (width 0.2) (layer "F.Cu") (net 13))
 (segment (start 99.314 149.86) (end 136.525 115.316) (width 0.2) (layer "F.Cu") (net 13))
 (via (at 122.682 169.672) (size 0.8) (drill 0.4) (layers "F.Cu" "B.Cu") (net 13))
 (segment (start 122.682 169.672) (end 125.349 169.037) (width 0.2) (layer "B.Cu") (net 13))
 (segment (start 130.175 169.291) (end 132.461 172.212) (width 0.2) (layer "B.Cu") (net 13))
 (segment (start 125.349 169.037) (end 130.175 169.291) (width 0.2) (layer "B.Cu") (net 13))
 (segment (start 124.587 174.879) (end 125.73 176.022) (width 0.2) (layer "F.Cu") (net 14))
 (segment (start 131.699 176.149) (end 132.461 174.752) (width 0.2) (layer "F.Cu") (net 14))
 (segment (start 124.46 172.339) (end 124.587 174.879) (width 0.2) (layer "F.Cu") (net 14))
 (segment (start 98.001705 147.28162) (end 97.79 154.813) (width 0.2) (layer "F.Cu") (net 14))
 (segment (start 125.73 176.022) (end 131.699 176.149) (width 0.2) (layer "F.Cu") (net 14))
 (segment (start 97.79 154.813) (end 124.46 172.339) (width 0.2) (layer "F.Cu") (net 14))
 (segment (start 116.967 5.207) (end 110.786295 3.21338) (width 0.2) (layer "F.Cu") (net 1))
 (segment (start 142.494 39.624) (end 142.621 35.306) (width 0.2) (layer "F.Cu") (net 1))
 (segment (start 99.949 154.051) (end 99.949 150.241) (width 0.2) (layer "F.Cu") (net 1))
 (segment (start 138.303 115.951) (end 138.049 110.363) (width 0.2) (layer "F.Cu") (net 1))
 (segment (start 138.049 110.363) (end 107.061 77.851) (width 0.2) (layer "F.Cu") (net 1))
 (segment (start 99.949 150.241) (end 138.303 115.951) (width 0.2) (layer "F.Cu") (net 1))
 (segment (start 107.442 70.231) (end 142.494 39.624) (width 0.2) (layer "F.Cu") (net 1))
 (segment (start 107.061 77.851) (end 107.442 70.231) (width 0.2) (layer "F.Cu") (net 1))
 (segment (start 124.714 170.053) (end 99.949 154.051) (width 0.2) (layer "F.Cu") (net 1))
 (segment (start 142.621 35.306) (end 116.967 5.207) (width 0.2) (layer "F.Cu") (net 1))
 (via (at 124.714 170.053) (size 0.8) (drill 0.4) (layers "F.Cu" "B.Cu") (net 1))
 (segment (start 124.714 170.053) (end 129.159 170.561) (width 0.2) (layer "B.Cu") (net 1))
 (segment (start 129.159 170.561) (end 129.921 172.212) (width 0.2) (layer "B.Cu") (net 1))
 (segment (start 128.651 168.275) (end 128.651 174.117) (width 0.2) (layer "F.Cu") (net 2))
 (segment (start 128.651 174.117) (end 129.921 174.752) (width 0.2) (layer "F.Cu") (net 2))
 (segment (start 104.859705 70.95462) (end 104.775 75.565) (width 0.2) (layer "F.Cu") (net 2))
 (via (at 128.651 168.275) (size 0.8) (drill 0.4) (layers "F.Cu" "B.Cu") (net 2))
 (via (at 104.775 75.565) (size 0.8) (drill 0.4) (layers "F.Cu" "B.Cu") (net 2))
 (segment (start 141.605 115.062) (end 140.843 112.776) (width 0.2) (layer "B.Cu") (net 2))
 (segment (start 99.314 149.86) (end 128.397 125.349) (width 0.2) (layer "B.Cu") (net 2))
 (segment (start 121.92 167.767) (end 99.568 152.908) (width 0.2) (layer "B.Cu") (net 2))
 (segment (start 137.16 110.49) (end 104.775 75.565) (width 0.2) (layer "B.Cu") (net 2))
 (segment (start 128.397 125.349) (end 140.97 115.824) (width 0.2) (layer "B.Cu") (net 2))
 (segment (start 140.97 115.824) (end 141.605 115.062) (width 0.2) (layer "B.Cu") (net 2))
 (segment (start 140.843 112.776) (end 137.16 110.49) (width 0.2) (layer "B.Cu") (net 2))
 (segment (start 99.568 152.908) (end 99.314 149.86) (width 0.2) (layer "B.Cu") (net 2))
 (segment (start 128.651 168.275) (end 121.92 167.767) (width 0.2) (layer "B.Cu") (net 2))
 (segment (start 138.938 116.459) (end 103.124 148.336) (width 0.2) (layer "F.Cu") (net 5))
 (segment (start 100.584 150.368) (end 100.584 153.924) (width 0.2) (layer "F.Cu") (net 5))
 (segment (start 103.124 148.336) (end 100.584 150.368) (width 0.2) (layer "F.Cu") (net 5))
 (segment (start 109.002 75.565) (end 110.744 79.121) (width 0.2) (layer "F.Cu") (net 5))
 (segment (start 110.744 79.121) (end 138.811 109.982) (width 0.2) (layer "F.Cu") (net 5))
 (segment (start 127.127 173.101) (end 127.381 172.212) (width 0.2) (layer "F.Cu") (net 5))
 (segment (start 100.584 153.924) (end 125.984 169.799) (width 0.2) (layer "F.Cu") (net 5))
 (segment (start 138.811 109.982) (end 138.938 116.459) (width 0.2) (layer "F.Cu") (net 5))
 (segment (start 125.984 169.799) (end 127.127 173.101) (width 0.2) (layer "F.Cu") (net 5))
 (segment (start 175.500422 79.121) (end 177.002 75.565) (width 0.2) (layer "F.Cu") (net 6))
 (segment (start 175.500422 79.121) (end 140.716 110.109) (width 0.2) (layer "F.Cu") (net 6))
 (segment (start 140.716 110.109) (end 140.462 114.046) (width 0.2) (layer "F.Cu") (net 6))
 (via (at 140.462 114.046) (size 0.8) (drill 0.4) (layers "F.Cu" "B.Cu") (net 6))
 (segment (start 140.462 114.046) (end 98.679 148.209) (width 0.2) (layer "B.Cu") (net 6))
 (segment (start 98.552 153.416) (end 125.222 172.593) (width 0.2) (layer "B.Cu") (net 6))
 (segment (start 98.679 148.209) (end 98.552 153.416) (width 0.2) (layer "B.Cu") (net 6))
 (segment (start 125.222 172.593) (end 127.381 174.752) (width 0.2) (layer "B.Cu") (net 6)))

